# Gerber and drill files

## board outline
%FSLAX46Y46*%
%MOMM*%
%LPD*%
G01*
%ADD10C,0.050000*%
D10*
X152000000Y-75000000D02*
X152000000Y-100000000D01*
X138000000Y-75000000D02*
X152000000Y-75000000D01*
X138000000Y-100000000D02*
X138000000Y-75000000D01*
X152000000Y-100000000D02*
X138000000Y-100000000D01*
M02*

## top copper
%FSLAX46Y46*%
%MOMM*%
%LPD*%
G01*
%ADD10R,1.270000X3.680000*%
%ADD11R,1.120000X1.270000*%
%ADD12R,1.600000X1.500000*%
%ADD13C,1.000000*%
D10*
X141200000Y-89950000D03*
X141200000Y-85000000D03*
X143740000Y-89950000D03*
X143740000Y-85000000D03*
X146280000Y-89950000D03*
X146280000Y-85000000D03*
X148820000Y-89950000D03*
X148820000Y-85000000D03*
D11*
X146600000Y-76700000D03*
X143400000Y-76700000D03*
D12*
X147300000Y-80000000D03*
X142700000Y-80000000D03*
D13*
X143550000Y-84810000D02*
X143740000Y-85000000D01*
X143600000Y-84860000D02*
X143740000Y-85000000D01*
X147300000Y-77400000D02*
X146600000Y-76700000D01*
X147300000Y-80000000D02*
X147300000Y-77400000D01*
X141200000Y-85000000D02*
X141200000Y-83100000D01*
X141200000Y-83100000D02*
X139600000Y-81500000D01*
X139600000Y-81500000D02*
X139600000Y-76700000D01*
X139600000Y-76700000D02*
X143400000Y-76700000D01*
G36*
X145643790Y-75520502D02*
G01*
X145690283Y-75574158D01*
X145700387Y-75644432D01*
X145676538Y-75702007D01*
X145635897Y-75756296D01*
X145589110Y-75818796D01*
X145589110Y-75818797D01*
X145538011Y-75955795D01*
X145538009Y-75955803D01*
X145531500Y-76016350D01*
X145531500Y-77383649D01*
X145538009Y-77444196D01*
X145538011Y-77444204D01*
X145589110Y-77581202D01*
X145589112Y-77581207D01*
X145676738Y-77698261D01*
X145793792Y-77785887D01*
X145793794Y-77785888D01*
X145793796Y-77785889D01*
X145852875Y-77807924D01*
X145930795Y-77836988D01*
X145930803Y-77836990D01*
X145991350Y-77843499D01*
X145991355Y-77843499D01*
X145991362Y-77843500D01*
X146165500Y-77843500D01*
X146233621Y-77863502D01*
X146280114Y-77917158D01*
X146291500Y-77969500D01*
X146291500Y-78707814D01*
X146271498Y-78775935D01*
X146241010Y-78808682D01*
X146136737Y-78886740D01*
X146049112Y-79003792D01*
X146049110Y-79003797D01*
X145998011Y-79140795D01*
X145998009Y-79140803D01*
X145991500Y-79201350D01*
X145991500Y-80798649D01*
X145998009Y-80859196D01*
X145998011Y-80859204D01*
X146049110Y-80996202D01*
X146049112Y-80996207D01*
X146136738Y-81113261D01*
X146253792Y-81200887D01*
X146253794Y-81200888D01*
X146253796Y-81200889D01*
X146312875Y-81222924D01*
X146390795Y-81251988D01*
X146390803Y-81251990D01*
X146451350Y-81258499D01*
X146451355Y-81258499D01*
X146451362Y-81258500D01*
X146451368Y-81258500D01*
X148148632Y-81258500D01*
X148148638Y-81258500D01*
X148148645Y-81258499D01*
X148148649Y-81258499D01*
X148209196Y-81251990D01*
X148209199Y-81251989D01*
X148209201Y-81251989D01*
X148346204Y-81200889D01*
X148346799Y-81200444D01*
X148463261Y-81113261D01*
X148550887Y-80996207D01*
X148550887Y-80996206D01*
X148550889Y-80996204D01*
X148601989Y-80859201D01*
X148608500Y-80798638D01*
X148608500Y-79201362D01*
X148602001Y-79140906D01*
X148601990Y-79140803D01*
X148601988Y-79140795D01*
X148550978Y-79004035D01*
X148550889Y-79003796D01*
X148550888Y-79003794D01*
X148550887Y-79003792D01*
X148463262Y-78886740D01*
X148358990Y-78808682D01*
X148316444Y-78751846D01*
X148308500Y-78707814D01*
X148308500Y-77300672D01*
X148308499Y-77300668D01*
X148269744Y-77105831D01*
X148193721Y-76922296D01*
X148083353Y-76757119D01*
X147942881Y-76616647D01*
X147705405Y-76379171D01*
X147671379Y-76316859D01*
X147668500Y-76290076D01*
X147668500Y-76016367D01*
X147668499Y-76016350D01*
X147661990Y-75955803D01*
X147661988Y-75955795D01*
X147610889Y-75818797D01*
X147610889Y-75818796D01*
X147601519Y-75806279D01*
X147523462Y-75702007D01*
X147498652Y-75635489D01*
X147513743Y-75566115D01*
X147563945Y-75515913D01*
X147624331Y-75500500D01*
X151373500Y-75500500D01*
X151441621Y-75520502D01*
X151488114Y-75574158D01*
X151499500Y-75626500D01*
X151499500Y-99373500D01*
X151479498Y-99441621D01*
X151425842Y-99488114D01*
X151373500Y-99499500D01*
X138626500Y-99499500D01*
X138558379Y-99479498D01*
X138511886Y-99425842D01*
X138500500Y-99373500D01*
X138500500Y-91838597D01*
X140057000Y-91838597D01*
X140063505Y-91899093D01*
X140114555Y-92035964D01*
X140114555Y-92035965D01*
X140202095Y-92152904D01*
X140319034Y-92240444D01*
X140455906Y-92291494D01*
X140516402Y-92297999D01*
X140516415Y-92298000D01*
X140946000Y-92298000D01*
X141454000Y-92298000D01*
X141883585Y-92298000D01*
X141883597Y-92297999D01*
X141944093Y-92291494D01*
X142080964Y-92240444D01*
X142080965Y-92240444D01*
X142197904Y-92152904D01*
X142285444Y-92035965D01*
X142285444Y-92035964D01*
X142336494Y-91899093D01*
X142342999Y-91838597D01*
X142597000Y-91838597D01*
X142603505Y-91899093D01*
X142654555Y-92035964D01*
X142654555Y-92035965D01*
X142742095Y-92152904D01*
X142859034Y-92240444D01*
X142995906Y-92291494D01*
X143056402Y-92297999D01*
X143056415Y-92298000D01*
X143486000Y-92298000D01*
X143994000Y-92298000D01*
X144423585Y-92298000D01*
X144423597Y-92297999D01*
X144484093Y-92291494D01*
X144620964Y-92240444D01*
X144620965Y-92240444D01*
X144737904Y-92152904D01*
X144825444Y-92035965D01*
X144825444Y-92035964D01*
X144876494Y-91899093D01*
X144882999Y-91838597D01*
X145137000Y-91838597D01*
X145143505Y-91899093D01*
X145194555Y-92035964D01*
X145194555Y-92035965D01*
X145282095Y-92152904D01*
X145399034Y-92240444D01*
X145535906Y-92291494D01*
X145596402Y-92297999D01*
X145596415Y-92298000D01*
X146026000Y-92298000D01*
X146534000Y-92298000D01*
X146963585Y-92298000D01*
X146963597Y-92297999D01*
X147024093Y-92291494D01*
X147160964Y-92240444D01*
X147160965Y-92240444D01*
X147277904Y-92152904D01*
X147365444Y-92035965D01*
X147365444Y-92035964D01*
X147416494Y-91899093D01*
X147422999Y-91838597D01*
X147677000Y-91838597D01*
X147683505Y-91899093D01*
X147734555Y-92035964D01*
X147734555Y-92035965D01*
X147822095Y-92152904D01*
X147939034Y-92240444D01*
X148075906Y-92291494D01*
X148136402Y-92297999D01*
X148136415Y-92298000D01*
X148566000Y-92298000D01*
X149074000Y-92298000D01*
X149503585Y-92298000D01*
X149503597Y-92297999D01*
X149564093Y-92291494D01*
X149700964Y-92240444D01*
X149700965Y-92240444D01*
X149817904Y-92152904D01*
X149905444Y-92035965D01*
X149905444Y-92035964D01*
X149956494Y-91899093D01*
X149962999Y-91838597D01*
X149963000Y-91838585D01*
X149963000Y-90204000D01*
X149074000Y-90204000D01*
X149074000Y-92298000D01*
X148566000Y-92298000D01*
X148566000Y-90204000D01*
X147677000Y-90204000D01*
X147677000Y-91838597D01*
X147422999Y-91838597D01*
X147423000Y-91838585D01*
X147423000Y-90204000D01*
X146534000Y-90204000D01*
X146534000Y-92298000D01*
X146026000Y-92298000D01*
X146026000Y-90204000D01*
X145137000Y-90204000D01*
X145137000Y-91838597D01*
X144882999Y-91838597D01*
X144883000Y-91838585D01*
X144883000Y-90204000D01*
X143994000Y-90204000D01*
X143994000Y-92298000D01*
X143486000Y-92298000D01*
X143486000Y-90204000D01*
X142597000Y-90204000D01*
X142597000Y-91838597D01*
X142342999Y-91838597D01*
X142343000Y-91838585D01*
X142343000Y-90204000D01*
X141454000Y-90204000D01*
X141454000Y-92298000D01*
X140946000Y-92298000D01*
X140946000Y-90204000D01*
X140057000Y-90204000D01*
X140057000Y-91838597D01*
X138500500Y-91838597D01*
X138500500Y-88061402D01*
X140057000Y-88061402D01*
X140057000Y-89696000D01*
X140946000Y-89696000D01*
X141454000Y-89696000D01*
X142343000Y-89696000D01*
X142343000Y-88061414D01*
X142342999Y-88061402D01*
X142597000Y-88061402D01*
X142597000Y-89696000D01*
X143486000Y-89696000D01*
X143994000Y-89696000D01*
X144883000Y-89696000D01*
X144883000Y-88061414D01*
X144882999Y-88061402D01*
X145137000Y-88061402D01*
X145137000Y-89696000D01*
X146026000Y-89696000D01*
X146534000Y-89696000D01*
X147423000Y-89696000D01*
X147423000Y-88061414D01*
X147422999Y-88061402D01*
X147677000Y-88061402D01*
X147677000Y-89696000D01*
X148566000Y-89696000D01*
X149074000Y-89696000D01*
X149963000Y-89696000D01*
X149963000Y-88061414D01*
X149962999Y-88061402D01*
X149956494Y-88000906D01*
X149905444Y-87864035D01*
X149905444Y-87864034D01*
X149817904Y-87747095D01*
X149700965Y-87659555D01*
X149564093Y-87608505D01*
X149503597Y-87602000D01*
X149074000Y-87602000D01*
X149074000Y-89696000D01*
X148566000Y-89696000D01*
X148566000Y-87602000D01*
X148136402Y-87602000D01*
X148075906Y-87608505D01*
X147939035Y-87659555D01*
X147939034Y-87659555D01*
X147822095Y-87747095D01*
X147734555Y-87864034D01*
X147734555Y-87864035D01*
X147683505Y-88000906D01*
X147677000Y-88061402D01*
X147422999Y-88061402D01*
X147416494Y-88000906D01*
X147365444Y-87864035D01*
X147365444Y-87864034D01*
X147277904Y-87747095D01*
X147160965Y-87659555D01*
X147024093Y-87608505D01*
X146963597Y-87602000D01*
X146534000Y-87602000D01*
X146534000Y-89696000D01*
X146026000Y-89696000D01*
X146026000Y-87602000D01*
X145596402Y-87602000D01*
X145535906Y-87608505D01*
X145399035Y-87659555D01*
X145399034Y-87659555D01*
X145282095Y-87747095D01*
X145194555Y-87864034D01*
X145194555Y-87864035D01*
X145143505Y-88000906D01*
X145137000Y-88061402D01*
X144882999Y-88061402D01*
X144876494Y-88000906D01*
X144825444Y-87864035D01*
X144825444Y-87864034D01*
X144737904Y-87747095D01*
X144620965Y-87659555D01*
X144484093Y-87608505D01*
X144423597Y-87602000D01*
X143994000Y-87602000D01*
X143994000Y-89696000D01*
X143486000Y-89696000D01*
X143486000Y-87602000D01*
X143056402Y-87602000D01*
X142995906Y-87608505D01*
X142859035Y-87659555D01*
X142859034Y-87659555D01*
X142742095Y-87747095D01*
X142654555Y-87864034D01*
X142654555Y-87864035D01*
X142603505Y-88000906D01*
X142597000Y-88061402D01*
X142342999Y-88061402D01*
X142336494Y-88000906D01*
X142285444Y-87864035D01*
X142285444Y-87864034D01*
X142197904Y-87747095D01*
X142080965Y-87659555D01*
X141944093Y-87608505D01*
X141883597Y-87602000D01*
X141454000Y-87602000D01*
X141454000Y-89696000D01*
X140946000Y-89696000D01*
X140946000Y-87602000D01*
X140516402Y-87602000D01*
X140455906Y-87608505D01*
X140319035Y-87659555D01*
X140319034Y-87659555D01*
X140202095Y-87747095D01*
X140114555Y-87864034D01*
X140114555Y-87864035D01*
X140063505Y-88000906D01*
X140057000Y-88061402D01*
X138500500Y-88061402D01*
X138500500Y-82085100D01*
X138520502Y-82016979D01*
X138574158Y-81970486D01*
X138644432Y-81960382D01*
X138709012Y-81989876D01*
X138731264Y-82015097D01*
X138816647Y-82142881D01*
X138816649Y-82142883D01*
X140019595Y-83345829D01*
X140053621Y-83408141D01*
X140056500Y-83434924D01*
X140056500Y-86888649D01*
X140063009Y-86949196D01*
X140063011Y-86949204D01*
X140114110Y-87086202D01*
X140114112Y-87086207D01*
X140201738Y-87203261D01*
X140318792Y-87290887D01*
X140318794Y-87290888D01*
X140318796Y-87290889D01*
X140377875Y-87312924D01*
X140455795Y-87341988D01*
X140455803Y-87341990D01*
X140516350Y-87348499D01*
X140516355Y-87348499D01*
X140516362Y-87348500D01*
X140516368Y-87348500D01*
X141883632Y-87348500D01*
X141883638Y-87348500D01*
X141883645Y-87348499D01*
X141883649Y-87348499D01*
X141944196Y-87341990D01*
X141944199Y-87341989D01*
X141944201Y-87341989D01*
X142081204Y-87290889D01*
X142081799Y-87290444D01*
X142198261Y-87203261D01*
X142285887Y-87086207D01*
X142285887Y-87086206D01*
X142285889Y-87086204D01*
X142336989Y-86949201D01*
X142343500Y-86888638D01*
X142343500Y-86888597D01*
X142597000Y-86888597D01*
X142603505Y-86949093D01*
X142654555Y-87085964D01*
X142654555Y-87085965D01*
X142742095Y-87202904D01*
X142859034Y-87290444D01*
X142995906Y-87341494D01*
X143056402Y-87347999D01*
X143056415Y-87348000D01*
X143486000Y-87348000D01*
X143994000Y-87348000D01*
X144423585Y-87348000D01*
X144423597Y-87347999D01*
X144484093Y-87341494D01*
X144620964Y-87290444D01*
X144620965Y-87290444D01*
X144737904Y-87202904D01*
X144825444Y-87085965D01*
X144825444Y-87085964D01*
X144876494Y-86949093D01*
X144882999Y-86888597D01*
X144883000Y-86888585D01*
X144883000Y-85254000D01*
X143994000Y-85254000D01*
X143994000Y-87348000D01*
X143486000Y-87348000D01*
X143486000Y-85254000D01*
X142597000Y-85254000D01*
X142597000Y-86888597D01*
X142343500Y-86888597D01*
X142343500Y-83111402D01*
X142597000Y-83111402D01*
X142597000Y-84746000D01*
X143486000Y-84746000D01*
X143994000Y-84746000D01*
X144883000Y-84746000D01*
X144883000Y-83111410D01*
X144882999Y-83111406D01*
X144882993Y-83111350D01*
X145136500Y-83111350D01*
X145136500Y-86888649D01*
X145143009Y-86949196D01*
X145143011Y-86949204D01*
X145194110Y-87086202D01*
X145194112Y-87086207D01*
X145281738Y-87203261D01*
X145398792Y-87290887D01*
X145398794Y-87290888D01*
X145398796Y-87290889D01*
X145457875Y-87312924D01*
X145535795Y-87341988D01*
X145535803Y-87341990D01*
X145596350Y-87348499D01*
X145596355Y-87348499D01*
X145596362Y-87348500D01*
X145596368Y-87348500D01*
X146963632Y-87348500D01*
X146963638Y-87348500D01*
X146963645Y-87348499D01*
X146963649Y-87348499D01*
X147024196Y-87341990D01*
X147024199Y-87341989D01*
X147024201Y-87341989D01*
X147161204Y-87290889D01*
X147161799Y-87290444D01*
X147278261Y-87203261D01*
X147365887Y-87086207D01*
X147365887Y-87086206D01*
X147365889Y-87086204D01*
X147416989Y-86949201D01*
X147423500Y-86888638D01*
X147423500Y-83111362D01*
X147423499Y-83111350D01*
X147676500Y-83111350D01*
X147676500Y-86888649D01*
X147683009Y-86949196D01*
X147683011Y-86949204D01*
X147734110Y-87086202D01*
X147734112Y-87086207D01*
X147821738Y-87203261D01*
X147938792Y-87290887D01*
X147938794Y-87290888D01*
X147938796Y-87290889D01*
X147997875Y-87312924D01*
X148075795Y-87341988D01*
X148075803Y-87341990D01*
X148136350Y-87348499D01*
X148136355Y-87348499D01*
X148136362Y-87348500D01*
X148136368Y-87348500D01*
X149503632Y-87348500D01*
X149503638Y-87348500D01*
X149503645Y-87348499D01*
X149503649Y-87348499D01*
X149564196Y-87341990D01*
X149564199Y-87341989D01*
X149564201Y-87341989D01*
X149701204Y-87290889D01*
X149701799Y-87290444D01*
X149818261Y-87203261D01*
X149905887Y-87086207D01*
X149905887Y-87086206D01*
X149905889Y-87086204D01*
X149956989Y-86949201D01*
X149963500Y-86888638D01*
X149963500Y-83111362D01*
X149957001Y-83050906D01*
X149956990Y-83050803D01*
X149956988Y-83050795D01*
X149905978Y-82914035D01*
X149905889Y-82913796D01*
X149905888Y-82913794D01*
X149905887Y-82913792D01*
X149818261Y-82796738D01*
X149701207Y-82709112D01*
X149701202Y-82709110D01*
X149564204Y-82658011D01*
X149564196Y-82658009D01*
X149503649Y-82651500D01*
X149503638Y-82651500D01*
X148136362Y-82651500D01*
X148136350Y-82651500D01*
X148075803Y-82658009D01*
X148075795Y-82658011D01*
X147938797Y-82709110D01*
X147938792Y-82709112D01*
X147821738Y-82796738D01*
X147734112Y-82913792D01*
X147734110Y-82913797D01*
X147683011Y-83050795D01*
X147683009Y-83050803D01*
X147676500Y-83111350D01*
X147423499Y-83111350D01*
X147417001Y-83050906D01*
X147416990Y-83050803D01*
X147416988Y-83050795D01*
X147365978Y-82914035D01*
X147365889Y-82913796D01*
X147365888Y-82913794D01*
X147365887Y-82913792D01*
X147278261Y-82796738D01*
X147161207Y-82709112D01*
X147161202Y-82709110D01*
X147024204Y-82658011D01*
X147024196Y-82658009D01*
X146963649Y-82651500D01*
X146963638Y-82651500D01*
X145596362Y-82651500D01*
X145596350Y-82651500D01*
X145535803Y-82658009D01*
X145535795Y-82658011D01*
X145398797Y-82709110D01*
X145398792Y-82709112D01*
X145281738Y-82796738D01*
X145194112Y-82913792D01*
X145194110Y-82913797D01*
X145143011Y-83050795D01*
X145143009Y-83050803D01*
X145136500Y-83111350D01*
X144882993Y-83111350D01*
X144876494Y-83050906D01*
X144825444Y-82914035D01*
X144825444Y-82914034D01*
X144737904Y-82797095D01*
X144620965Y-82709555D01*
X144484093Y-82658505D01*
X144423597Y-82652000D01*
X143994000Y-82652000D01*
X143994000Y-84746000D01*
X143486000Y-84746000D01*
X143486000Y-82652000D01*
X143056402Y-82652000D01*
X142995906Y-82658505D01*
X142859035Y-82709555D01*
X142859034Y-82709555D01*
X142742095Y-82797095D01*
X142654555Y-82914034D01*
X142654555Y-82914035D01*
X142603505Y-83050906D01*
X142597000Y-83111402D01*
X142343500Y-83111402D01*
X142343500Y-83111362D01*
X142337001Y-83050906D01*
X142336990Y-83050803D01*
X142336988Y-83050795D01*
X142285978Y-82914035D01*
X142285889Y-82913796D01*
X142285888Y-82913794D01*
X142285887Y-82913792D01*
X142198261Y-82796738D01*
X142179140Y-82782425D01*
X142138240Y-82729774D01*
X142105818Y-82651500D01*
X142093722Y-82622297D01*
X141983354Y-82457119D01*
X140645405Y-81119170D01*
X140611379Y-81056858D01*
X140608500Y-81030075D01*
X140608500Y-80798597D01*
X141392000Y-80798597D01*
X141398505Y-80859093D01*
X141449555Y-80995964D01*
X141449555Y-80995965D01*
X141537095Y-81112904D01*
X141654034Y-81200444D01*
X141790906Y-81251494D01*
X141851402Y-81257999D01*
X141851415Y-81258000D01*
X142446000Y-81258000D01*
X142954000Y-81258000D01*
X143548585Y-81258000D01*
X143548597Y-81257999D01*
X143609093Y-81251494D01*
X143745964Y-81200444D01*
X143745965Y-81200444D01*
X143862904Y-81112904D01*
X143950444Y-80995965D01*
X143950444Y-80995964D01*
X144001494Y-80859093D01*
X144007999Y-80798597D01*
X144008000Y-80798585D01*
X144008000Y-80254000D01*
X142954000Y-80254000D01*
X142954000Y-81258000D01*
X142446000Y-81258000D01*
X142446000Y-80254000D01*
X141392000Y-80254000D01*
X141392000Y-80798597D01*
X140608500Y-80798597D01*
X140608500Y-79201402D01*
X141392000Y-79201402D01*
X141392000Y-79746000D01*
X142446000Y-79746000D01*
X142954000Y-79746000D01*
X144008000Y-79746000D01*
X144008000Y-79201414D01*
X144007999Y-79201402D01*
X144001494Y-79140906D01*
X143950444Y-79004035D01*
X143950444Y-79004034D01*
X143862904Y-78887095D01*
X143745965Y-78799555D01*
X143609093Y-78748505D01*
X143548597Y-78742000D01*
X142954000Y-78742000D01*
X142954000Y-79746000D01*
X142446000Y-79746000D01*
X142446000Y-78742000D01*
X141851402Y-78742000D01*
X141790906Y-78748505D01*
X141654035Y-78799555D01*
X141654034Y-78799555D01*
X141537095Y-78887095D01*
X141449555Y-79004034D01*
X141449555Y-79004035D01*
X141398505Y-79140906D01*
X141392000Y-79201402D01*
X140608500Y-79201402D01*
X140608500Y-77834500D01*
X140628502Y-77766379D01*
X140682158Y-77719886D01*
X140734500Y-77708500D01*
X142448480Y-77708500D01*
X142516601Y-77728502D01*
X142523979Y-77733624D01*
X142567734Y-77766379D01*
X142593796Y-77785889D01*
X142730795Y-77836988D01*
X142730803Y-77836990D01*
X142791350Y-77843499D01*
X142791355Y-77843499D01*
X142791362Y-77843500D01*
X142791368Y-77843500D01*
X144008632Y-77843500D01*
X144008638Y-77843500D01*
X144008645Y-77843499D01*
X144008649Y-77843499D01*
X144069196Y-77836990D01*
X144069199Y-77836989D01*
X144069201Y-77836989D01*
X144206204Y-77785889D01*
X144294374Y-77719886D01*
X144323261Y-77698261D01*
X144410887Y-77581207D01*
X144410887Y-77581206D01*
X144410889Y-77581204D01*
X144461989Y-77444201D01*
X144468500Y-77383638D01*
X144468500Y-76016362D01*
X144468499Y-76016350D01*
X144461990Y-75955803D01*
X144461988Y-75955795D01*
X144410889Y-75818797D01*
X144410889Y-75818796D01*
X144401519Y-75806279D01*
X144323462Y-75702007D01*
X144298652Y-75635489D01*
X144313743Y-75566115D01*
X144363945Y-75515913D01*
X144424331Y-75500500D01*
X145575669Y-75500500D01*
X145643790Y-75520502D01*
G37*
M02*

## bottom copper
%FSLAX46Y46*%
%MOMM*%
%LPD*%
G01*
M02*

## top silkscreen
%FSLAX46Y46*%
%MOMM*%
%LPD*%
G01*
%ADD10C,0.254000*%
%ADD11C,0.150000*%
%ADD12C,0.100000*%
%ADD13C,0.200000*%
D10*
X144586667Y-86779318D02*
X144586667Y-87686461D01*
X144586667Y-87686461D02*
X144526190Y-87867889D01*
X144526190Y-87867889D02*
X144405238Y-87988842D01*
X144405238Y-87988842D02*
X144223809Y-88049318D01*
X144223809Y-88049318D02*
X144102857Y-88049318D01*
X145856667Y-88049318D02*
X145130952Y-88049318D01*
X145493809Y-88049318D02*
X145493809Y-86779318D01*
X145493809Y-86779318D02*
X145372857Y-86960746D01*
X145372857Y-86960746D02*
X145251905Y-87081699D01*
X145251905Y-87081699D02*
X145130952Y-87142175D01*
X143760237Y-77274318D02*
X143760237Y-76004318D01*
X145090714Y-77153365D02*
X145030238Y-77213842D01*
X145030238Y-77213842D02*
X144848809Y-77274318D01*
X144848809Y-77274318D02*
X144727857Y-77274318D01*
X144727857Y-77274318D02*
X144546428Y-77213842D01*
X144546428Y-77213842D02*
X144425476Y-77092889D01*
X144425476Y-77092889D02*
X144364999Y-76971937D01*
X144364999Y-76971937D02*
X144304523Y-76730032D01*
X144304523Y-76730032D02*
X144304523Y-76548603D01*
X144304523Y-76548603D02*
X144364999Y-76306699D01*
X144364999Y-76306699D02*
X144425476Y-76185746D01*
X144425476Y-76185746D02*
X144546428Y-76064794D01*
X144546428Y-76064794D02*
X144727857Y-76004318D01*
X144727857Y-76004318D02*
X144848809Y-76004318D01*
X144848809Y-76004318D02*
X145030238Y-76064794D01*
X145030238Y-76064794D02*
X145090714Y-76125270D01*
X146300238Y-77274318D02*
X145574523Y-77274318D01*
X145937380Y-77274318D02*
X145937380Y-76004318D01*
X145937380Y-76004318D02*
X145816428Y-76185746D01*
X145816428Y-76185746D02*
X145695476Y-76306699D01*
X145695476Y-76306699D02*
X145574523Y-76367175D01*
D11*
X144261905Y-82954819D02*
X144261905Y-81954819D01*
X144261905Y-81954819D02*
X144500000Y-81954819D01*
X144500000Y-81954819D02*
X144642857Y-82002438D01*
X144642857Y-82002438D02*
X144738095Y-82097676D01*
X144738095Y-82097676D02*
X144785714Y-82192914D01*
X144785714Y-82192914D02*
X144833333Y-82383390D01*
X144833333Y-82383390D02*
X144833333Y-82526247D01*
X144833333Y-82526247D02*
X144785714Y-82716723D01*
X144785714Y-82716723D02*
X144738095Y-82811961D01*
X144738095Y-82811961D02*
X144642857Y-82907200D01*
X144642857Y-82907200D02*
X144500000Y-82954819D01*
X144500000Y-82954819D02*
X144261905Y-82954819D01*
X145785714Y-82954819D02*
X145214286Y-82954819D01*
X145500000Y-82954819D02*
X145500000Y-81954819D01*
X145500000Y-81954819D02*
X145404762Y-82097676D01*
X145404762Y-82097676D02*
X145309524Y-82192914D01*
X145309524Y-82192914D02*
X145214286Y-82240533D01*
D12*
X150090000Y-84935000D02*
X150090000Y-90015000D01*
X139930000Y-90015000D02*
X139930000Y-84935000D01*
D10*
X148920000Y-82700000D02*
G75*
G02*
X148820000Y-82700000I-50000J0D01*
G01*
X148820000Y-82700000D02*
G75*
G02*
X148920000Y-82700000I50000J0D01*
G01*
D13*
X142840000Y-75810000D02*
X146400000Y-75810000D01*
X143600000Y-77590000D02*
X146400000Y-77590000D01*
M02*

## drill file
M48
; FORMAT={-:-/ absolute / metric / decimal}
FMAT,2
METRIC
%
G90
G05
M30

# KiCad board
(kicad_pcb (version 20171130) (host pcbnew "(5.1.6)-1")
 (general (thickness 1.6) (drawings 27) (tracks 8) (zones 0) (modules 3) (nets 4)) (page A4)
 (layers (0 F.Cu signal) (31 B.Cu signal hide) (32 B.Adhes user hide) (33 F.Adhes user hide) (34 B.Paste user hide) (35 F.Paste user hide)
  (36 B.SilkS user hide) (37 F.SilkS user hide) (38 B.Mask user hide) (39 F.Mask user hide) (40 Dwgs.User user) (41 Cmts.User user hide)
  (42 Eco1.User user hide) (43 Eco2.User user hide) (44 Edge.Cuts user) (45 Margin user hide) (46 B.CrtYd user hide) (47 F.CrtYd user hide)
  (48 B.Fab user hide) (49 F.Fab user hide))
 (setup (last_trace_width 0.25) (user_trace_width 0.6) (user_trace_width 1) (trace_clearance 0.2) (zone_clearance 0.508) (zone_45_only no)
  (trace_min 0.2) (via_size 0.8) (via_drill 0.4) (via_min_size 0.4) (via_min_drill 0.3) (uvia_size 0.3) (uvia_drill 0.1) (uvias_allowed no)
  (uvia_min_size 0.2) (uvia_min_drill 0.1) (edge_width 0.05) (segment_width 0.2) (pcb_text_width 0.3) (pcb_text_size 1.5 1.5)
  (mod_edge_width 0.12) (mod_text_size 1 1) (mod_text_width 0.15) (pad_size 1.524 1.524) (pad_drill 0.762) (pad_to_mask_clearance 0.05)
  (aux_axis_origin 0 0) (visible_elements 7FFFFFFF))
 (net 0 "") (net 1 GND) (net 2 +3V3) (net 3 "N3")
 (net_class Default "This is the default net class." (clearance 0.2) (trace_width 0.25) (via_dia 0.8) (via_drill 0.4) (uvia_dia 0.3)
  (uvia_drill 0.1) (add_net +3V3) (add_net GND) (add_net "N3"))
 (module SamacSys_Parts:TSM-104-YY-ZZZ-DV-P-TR (layer F.Cu) (at 145.01 87.475)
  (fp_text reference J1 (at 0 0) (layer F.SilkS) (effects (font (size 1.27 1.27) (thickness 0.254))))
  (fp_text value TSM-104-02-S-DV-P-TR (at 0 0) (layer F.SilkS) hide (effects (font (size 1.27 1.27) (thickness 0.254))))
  (fp_line (start 5.08 -2.54) (end 5.08 2.54) (layer F.SilkS) (width 0.1))
  (fp_line (start -5.08 2.54) (end -5.08 -2.54) (layer F.SilkS) (width 0.1))
  (fp_circle (center 3.86 -4.775) (end 3.81 -4.775) (layer F.SilkS) (width 0.254))
  (pad 8 smd rect (at -3.81 2.475) (size 1.27 3.68) (layers F.Cu F.Paste F.Mask) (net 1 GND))
  (pad 7 smd rect (at -3.81 -2.475) (size 1.27 3.68) (layers F.Cu F.Paste F.Mask) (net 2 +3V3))
  (pad 6 smd rect (at -1.27 2.475) (size 1.27 3.68) (layers F.Cu F.Paste F.Mask) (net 1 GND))
  (pad 5 smd rect (at -1.27 -2.475) (size 1.27 3.68) (layers F.Cu F.Paste F.Mask) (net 1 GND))
  (pad 4 smd rect (at 1.27 2.475) (size 1.27 3.68) (layers F.Cu F.Paste F.Mask) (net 1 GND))
  (pad 3 smd rect (at 1.27 -2.475) (size 1.27 3.68) (layers F.Cu F.Paste F.Mask))
  (pad 2 smd rect (at 3.81 2.475) (size 1.27 3.68) (layers F.Cu F.Paste F.Mask) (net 1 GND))
  (pad 1 smd rect (at 3.81 -2.475) (size 1.27 3.68) (layers F.Cu F.Paste F.Mask)))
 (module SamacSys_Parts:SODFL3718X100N (layer F.Cu) (at 145 76.7)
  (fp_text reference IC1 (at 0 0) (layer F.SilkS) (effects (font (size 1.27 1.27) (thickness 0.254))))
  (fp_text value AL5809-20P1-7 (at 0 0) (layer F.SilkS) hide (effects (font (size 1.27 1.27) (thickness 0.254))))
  (fp_line (start -2.16 -0.89) (end 1.4 -0.89) (layer F.SilkS) (width 0.2))
  (fp_line (start -1.4 0.89) (end 1.4 0.89) (layer F.SilkS) (width 0.2))
  (pad 2 smd rect (at 1.6 0) (size 1.12 1.27) (layers F.Cu F.Paste F.Mask) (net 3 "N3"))
  (pad 1 smd rect (at -1.6 0) (size 1.12 1.27) (layers F.Cu F.Paste F.Mask) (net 2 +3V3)))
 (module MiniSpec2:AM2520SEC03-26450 (layer F.Cu) (at 145 80)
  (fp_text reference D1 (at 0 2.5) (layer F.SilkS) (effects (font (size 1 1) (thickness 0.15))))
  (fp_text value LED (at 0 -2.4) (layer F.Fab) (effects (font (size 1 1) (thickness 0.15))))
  (pad 2 smd rect (at 2.3 0) (size 1.6 1.5) (layers F.Cu F.Paste F.Mask) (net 3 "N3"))
  (pad 1 smd rect (at -2.3 0) (size 1.6 1.5) (layers F.Cu F.Paste F.Mask) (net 1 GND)))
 (gr_line (start 152 75) (end 152 100) (layer Edge.Cuts) (width 0.05))
 (gr_line (start 138 75) (end 152 75) (layer Edge.Cuts) (width 0.05))
 (gr_line (start 138 100) (end 138 75) (layer Edge.Cuts) (width 0.05))
 (gr_line (start 152 100) (end 138 100) (layer Edge.Cuts) (width 0.05))
 (segment (start 143.55 84.81) (end 143.74 85) (width 1) (layer F.Cu) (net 1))
 (segment (start 143.6 84.86) (end 143.74 85) (width 1) (layer F.Cu) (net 1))
 (segment (start 147.3 77.4) (end 146.6 76.7) (width 1) (layer F.Cu) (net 3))
 (segment (start 147.3 80) (end 147.3 77.4) (width 1) (layer F.Cu) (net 3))
 (segment (start 141.2 85) (end 141.2 83.1) (width 1) (layer F.Cu) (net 2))
 (segment (start 141.2 83.1) (end 139.6 81.5) (width 1) (layer F.Cu) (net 2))
 (segment (start 139.6 81.5) (end 139.6 76.7) (width 1) (layer F.Cu) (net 2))
 (segment (start 139.6 76.7) (end 143.4 76.7) (width 1) (layer F.Cu) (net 2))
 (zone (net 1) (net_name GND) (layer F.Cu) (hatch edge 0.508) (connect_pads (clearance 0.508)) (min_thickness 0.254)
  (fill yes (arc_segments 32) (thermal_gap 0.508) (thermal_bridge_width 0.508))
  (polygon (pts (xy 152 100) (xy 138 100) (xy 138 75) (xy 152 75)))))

